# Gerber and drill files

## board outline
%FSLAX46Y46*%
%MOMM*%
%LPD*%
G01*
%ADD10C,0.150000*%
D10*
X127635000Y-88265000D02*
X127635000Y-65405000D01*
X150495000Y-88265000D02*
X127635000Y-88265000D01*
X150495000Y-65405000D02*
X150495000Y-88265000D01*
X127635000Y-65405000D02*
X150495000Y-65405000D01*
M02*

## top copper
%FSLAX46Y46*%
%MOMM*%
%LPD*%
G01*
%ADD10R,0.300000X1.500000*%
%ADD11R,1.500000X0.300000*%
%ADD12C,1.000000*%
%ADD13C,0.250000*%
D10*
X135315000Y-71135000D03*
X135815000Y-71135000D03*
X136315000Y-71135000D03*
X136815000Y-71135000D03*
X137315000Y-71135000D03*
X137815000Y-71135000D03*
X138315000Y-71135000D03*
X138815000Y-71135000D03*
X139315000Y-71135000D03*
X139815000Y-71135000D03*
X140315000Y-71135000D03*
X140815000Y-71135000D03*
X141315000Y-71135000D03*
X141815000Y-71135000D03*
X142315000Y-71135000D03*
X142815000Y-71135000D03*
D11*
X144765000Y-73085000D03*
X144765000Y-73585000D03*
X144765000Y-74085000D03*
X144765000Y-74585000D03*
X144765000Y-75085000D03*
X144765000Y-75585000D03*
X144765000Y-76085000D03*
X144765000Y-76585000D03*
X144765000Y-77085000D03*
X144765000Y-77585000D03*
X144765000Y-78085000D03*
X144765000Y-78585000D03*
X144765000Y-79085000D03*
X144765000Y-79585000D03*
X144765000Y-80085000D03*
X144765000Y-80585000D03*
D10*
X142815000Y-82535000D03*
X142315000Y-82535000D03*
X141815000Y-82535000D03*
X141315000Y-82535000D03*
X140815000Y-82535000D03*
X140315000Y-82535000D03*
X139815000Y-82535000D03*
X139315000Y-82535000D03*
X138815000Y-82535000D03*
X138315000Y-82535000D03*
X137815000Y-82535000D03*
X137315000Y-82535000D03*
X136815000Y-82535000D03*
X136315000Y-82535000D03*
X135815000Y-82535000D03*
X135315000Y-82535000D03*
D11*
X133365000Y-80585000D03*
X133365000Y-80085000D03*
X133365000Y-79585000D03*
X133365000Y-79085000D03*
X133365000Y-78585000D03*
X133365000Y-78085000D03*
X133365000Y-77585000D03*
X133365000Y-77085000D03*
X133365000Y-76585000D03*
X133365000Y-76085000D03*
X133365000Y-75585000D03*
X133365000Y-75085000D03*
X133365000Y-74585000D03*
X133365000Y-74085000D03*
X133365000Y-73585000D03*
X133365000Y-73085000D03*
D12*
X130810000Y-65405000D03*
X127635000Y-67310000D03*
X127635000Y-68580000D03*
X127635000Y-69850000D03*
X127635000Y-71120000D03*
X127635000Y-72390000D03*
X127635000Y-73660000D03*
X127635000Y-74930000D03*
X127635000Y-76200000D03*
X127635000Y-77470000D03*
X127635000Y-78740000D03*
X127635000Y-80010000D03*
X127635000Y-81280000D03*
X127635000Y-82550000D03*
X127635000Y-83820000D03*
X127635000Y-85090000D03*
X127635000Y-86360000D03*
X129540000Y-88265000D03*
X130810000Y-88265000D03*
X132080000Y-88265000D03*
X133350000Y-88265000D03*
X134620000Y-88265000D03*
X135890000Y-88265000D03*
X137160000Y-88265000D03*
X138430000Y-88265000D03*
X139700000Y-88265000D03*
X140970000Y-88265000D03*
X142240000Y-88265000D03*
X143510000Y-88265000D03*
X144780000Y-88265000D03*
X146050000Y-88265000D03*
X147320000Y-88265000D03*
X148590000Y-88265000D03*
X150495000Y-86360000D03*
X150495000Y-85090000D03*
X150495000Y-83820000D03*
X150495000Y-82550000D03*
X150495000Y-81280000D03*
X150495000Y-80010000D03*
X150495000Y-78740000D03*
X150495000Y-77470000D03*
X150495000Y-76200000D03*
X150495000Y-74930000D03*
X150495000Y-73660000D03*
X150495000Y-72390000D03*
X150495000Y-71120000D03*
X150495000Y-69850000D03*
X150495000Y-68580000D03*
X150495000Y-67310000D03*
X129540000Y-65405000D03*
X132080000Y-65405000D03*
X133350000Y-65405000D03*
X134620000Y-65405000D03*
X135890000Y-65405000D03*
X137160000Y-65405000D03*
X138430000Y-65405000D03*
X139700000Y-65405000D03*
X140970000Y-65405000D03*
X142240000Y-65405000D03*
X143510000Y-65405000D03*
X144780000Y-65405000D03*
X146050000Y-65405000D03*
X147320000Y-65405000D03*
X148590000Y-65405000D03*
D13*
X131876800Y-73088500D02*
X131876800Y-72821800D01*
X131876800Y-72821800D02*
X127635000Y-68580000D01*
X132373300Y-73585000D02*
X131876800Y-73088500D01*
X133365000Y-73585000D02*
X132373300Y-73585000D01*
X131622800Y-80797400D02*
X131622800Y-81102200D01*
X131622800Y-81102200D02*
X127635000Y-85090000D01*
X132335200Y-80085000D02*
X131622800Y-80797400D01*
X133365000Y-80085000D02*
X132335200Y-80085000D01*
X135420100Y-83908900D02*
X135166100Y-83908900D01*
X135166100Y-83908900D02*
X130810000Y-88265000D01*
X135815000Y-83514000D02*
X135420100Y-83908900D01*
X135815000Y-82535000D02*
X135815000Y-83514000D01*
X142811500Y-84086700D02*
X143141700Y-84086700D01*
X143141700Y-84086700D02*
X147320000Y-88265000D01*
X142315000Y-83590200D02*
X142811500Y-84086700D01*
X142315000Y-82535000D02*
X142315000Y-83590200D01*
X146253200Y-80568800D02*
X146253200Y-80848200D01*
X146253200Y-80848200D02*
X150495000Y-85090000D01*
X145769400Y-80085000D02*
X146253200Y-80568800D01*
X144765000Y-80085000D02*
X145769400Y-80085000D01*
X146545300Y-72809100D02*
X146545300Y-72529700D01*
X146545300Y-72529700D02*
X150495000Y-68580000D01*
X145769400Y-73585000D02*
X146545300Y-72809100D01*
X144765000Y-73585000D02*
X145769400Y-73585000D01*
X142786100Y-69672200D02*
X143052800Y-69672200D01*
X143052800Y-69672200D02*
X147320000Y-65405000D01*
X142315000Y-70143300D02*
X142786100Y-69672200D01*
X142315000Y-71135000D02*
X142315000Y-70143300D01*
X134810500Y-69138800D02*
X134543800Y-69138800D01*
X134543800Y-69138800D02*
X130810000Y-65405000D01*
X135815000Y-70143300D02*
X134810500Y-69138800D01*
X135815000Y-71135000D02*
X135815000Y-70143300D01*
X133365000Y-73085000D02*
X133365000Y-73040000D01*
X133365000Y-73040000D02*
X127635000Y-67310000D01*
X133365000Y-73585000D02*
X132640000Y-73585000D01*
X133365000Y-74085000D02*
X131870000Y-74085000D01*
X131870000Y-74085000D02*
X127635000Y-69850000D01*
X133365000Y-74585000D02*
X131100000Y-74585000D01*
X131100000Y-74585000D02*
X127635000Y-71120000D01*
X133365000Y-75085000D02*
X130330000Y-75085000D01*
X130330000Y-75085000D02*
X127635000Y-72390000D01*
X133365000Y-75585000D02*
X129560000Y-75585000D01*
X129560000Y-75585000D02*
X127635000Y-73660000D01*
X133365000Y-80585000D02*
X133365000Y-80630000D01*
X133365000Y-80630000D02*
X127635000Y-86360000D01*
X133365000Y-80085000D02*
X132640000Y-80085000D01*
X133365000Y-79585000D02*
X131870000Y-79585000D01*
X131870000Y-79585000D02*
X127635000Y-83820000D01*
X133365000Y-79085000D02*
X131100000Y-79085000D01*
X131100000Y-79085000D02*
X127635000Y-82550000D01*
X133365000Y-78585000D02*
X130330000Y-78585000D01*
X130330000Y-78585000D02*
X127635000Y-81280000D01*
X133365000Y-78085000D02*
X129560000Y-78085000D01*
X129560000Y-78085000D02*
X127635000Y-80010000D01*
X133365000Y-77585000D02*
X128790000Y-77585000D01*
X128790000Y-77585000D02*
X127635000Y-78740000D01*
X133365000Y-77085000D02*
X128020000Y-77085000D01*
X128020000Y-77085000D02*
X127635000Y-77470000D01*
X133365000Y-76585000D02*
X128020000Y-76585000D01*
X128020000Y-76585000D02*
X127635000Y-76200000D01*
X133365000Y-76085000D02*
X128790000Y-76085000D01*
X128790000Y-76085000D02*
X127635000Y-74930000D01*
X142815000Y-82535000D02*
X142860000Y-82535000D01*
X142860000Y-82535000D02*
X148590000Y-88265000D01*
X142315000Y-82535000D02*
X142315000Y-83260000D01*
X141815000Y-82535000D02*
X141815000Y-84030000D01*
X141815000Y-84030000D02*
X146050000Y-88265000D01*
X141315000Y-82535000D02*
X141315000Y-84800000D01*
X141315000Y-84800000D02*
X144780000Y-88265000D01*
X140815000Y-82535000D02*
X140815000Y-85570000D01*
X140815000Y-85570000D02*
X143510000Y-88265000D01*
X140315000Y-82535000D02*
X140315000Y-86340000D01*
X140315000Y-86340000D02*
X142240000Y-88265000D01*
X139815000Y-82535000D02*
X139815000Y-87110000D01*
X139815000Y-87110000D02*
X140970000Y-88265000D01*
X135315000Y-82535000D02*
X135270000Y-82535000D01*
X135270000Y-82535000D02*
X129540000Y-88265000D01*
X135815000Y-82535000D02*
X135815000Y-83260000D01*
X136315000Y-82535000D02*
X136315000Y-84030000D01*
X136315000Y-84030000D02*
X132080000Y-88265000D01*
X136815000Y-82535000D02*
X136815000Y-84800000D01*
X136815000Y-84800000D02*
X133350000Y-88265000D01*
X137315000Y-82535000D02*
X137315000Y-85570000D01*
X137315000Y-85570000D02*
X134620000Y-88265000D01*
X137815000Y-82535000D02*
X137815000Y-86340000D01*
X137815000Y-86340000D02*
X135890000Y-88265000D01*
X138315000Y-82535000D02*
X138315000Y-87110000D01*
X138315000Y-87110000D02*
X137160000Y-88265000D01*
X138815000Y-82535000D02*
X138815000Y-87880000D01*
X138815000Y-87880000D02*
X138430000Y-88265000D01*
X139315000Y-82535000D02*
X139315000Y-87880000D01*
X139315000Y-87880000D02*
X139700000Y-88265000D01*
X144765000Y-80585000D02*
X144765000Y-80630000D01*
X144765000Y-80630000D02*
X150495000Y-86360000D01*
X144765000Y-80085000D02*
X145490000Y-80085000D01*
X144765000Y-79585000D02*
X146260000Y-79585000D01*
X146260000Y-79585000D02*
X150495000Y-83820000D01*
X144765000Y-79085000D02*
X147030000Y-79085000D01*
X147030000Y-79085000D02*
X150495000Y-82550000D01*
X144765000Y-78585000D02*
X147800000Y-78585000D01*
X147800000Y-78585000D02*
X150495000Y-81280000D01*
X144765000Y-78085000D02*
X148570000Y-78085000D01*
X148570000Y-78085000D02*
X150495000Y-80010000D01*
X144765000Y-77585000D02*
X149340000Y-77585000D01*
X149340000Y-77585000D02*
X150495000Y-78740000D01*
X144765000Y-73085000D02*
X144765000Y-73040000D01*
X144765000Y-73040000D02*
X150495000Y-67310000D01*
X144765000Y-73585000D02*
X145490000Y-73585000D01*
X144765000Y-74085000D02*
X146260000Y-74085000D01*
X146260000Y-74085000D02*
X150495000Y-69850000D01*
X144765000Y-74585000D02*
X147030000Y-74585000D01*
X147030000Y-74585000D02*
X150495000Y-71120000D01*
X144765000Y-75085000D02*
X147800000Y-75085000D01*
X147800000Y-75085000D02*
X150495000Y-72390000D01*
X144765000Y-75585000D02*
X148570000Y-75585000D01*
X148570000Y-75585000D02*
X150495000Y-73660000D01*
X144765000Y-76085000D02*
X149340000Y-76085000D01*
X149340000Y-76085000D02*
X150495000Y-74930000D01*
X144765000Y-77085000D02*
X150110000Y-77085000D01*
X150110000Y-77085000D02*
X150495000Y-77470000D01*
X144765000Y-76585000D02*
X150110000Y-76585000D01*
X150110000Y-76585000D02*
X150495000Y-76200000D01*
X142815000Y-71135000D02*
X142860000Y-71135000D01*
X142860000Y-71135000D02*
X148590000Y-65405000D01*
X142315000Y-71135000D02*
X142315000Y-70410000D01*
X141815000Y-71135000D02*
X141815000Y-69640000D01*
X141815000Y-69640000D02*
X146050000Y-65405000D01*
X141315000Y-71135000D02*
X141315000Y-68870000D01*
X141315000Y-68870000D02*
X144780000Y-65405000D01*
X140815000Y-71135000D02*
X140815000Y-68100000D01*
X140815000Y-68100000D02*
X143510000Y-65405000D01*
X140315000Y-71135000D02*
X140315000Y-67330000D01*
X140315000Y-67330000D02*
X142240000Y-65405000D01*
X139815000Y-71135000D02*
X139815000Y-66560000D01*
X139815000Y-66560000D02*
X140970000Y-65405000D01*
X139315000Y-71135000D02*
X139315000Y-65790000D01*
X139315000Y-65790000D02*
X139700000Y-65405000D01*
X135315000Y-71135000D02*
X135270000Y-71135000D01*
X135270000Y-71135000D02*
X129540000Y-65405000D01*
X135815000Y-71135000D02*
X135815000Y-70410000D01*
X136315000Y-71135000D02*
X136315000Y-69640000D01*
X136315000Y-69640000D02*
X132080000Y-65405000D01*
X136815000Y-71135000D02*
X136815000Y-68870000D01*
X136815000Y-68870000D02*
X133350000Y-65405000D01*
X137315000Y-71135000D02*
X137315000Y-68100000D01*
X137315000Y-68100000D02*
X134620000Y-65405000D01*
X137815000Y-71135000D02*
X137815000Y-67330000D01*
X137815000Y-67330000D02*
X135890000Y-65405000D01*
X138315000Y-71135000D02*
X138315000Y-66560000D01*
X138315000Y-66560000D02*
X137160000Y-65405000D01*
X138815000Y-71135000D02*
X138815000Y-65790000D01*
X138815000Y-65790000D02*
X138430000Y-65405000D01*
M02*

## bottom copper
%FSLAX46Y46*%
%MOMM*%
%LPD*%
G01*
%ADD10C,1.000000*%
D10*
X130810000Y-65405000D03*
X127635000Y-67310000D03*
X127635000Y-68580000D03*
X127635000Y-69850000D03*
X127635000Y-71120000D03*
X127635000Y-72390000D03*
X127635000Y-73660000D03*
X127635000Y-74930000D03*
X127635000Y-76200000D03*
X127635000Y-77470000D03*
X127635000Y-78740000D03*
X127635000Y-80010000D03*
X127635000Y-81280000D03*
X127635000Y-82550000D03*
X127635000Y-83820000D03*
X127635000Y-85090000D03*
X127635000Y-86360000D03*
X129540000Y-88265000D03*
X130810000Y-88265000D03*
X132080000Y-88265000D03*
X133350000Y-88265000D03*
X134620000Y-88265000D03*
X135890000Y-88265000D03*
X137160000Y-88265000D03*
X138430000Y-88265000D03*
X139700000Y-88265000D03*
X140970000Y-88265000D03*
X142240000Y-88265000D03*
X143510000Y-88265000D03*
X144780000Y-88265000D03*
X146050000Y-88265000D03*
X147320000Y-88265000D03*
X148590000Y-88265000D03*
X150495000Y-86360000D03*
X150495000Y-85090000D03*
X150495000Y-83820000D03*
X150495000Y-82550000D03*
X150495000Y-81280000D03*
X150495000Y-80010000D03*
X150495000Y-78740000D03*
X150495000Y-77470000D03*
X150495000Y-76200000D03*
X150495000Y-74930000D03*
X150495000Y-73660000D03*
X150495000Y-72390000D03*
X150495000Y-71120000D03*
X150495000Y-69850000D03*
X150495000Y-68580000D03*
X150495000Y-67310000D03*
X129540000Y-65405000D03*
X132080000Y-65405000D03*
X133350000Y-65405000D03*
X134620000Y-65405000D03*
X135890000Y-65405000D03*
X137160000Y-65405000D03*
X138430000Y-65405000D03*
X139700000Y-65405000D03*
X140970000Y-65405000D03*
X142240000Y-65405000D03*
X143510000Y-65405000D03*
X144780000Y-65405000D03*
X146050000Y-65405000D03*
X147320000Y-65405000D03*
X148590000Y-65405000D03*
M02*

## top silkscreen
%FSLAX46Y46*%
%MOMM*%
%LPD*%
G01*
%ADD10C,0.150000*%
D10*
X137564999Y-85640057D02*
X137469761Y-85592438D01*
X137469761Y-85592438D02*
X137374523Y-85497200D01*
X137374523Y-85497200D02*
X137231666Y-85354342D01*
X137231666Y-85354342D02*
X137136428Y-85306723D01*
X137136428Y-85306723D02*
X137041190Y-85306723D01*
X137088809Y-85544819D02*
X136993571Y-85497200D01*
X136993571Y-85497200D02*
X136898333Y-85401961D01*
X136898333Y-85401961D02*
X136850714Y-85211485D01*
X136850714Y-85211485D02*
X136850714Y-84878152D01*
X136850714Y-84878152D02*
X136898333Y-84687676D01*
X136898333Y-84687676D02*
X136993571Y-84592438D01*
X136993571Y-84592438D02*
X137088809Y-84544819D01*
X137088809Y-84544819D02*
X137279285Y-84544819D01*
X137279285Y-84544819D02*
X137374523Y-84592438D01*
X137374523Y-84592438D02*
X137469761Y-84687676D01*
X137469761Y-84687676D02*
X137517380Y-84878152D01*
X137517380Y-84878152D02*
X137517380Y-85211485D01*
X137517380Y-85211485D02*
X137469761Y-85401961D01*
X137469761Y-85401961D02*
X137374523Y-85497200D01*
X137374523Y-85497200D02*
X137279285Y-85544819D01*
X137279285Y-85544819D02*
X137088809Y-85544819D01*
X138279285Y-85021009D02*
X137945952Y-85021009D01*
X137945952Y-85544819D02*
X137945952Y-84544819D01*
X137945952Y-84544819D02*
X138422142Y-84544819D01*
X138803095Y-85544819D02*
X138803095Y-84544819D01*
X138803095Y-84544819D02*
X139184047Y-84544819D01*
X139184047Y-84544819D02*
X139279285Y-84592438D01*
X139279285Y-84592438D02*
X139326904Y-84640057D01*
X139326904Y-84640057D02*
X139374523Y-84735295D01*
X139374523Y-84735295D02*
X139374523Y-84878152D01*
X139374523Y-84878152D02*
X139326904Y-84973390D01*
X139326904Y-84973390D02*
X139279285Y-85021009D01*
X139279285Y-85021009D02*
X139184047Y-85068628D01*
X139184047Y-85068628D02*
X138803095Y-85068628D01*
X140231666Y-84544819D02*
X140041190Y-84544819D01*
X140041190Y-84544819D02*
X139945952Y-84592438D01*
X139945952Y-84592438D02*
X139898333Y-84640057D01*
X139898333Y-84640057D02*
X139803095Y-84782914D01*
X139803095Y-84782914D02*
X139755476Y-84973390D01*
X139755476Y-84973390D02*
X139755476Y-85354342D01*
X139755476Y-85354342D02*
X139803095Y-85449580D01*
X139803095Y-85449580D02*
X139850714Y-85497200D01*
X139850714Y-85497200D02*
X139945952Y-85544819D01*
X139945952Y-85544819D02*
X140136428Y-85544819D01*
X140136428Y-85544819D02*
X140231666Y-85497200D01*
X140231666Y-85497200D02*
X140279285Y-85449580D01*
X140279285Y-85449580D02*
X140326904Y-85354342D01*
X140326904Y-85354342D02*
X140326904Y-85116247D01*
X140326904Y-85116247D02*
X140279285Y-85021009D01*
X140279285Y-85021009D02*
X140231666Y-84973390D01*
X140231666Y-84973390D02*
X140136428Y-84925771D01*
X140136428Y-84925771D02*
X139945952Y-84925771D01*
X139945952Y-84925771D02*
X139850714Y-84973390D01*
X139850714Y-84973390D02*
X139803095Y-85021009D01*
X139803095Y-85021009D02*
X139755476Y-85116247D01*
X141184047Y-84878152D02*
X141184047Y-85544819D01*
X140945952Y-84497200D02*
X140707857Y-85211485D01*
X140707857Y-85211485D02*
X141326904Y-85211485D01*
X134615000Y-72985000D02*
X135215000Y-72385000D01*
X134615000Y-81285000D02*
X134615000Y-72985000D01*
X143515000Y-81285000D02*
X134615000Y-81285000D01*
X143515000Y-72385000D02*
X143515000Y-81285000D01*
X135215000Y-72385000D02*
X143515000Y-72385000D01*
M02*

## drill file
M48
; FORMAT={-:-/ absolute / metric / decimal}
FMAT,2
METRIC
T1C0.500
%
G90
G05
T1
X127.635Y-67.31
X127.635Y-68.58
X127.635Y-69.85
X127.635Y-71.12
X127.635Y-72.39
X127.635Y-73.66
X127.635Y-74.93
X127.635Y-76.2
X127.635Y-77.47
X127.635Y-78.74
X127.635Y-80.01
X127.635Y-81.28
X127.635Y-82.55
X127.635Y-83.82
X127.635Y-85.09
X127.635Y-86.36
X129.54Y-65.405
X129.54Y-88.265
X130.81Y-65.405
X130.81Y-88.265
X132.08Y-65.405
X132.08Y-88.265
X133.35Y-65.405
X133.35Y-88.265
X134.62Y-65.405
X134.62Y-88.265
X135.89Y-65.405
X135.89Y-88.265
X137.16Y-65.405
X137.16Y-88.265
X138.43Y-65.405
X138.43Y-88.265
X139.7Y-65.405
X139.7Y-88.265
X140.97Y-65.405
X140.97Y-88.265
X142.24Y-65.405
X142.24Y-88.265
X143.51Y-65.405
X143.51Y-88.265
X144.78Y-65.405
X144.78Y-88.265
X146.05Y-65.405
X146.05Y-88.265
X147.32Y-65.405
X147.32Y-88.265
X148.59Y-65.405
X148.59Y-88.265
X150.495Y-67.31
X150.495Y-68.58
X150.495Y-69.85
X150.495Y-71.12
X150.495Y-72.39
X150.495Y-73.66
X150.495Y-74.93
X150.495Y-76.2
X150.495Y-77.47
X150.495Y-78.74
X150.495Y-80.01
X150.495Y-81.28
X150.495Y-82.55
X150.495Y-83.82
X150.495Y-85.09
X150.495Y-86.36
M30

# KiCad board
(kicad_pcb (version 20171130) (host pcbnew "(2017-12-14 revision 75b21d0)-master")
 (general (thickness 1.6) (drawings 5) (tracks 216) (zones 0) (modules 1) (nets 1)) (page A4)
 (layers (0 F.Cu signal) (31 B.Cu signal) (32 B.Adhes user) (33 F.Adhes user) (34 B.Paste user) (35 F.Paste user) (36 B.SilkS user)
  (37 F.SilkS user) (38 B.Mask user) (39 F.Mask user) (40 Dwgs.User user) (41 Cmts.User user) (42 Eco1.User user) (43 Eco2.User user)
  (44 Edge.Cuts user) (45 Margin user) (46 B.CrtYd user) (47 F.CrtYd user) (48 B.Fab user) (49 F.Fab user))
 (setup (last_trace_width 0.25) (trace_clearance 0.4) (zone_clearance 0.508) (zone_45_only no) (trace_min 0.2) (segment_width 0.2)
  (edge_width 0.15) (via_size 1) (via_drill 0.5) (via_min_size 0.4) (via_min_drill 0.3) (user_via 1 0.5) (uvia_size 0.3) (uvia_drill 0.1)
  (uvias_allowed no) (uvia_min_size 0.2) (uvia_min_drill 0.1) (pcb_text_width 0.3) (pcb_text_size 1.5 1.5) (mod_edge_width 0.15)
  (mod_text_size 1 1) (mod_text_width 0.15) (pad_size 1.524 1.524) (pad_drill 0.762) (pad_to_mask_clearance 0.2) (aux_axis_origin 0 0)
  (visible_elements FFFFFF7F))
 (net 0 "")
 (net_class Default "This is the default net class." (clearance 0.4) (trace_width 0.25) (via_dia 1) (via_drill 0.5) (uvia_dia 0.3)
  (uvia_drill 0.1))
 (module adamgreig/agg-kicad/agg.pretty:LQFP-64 (layer F.Cu) (at 139.065 76.835)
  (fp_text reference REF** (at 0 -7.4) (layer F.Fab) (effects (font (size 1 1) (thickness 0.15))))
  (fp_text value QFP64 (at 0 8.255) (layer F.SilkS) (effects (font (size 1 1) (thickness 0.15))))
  (fp_line (start -4.45 -3.85) (end -3.85 -4.45) (layer F.SilkS) (width 0.15))
  (fp_line (start -4.45 4.45) (end -4.45 -3.85) (layer F.SilkS) (width 0.15))
  (fp_line (start 4.45 4.45) (end -4.45 4.45) (layer F.SilkS) (width 0.15))
  (fp_line (start 4.45 -4.45) (end 4.45 4.45) (layer F.SilkS) (width 0.15))
  (fp_line (start -3.85 -4.45) (end 4.45 -4.45) (layer F.SilkS) (width 0.15))
  (pad 64 smd rect (at -3.75 -5.7) (size 0.3 1.5) (layers F.Cu F.Paste F.Mask))
  (pad 63 smd rect (at -3.25 -5.7) (size 0.3 1.5) (layers F.Cu F.Paste F.Mask))
  (pad 62 smd rect (at -2.75 -5.7) (size 0.3 1.5) (layers F.Cu F.Paste F.Mask))
  (pad 61 smd rect (at -2.25 -5.7) (size 0.3 1.5) (layers F.Cu F.Paste F.Mask))
  (pad 60 smd rect (at -1.75 -5.7) (size 0.3 1.5) (layers F.Cu F.Paste F.Mask))
  (pad 59 smd rect (at -1.25 -5.7) (size 0.3 1.5) (layers F.Cu F.Paste F.Mask))
  (pad 58 smd rect (at -0.75 -5.7) (size 0.3 1.5) (layers F.Cu F.Paste F.Mask))
  (pad 57 smd rect (at -0.25 -5.7) (size 0.3 1.5) (layers F.Cu F.Paste F.Mask))
  (pad 56 smd rect (at 0.25 -5.7) (size 0.3 1.5) (layers F.Cu F.Paste F.Mask))
  (pad 55 smd rect (at 0.75 -5.7) (size 0.3 1.5) (layers F.Cu F.Paste F.Mask))
  (pad 54 smd rect (at 1.25 -5.7) (size 0.3 1.5) (layers F.Cu F.Paste F.Mask))
  (pad 53 smd rect (at 1.75 -5.7) (size 0.3 1.5) (layers F.Cu F.Paste F.Mask))
  (pad 52 smd rect (at 2.25 -5.7) (size 0.3 1.5) (layers F.Cu F.Paste F.Mask))
  (pad 51 smd rect (at 2.75 -5.7) (size 0.3 1.5) (layers F.Cu F.Paste F.Mask))
  (pad 50 smd rect (at 3.25 -5.7) (size 0.3 1.5) (layers F.Cu F.Paste F.Mask))
  (pad 49 smd rect (at 3.75 -5.7) (size 0.3 1.5) (layers F.Cu F.Paste F.Mask))
  (pad 48 smd rect (at 5.7 -3.75) (size 1.5 0.3) (layers F.Cu F.Paste F.Mask))
  (pad 47 smd rect (at 5.7 -3.25) (size 1.5 0.3) (layers F.Cu F.Paste F.Mask))
  (pad 46 smd rect (at 5.7 -2.75) (size 1.5 0.3) (layers F.Cu F.Paste F.Mask))
  (pad 45 smd rect (at 5.7 -2.25) (size 1.5 0.3) (layers F.Cu F.Paste F.Mask))
  (pad 44 smd rect (at 5.7 -1.75) (size 1.5 0.3) (layers F.Cu F.Paste F.Mask))
  (pad 43 smd rect (at 5.7 -1.25) (size 1.5 0.3) (layers F.Cu F.Paste F.Mask))
  (pad 42 smd rect (at 5.7 -0.75) (size 1.5 0.3) (layers F.Cu F.Paste F.Mask))
  (pad 41 smd rect (at 5.7 -0.25) (size 1.5 0.3) (layers F.Cu F.Paste F.Mask))
  (pad 40 smd rect (at 5.7 0.25) (size 1.5 0.3) (layers F.Cu F.Paste F.Mask))
  (pad 39 smd rect (at 5.7 0.75) (size 1.5 0.3) (layers F.Cu F.Paste F.Mask))
  (pad 38 smd rect (at 5.7 1.25) (size 1.5 0.3) (layers F.Cu F.Paste F.Mask))
  (pad 37 smd rect (at 5.7 1.75) (size 1.5 0.3) (layers F.Cu F.Paste F.Mask))
  (pad 36 smd rect (at 5.7 2.25) (size 1.5 0.3) (layers F.Cu F.Paste F.Mask))
  (pad 35 smd rect (at 5.7 2.75) (size 1.5 0.3) (layers F.Cu F.Paste F.Mask))
  (pad 34 smd rect (at 5.7 3.25) (size 1.5 0.3) (layers F.Cu F.Paste F.Mask))
  (pad 33 smd rect (at 5.7 3.75) (size 1.5 0.3) (layers F.Cu F.Paste F.Mask))
  (pad 32 smd rect (at 3.75 5.7) (size 0.3 1.5) (layers F.Cu F.Paste F.Mask))
  (pad 31 smd rect (at 3.25 5.7) (size 0.3 1.5) (layers F.Cu F.Paste F.Mask))
  (pad 30 smd rect (at 2.75 5.7) (size 0.3 1.5) (layers F.Cu F.Paste F.Mask))
  (pad 29 smd rect (at 2.25 5.7) (size 0.3 1.5) (layers F.Cu F.Paste F.Mask))
  (pad 28 smd rect (at 1.75 5.7) (size 0.3 1.5) (layers F.Cu F.Paste F.Mask))
  (pad 27 smd rect (at 1.25 5.7) (size 0.3 1.5) (layers F.Cu F.Paste F.Mask))
  (pad 26 smd rect (at 0.75 5.7) (size 0.3 1.5) (layers F.Cu F.Paste F.Mask))
  (pad 25 smd rect (at 0.25 5.7) (size 0.3 1.5) (layers F.Cu F.Paste F.Mask))
  (pad 24 smd rect (at -0.25 5.7) (size 0.3 1.5) (layers F.Cu F.Paste F.Mask))
  (pad 23 smd rect (at -0.75 5.7) (size 0.3 1.5) (layers F.Cu F.Paste F.Mask))
  (pad 22 smd rect (at -1.25 5.7) (size 0.3 1.5) (layers F.Cu F.Paste F.Mask))
  (pad 21 smd rect (at -1.75 5.7) (size 0.3 1.5) (layers F.Cu F.Paste F.Mask))
  (pad 20 smd rect (at -2.25 5.7) (size 0.3 1.5) (layers F.Cu F.Paste F.Mask))
  (pad 19 smd rect (at -2.75 5.7) (size 0.3 1.5) (layers F.Cu F.Paste F.Mask))
  (pad 18 smd rect (at -3.25 5.7) (size 0.3 1.5) (layers F.Cu F.Paste F.Mask))
  (pad 17 smd rect (at -3.75 5.7) (size 0.3 1.5) (layers F.Cu F.Paste F.Mask))
  (pad 16 smd rect (at -5.7 3.75) (size 1.5 0.3) (layers F.Cu F.Paste F.Mask))
  (pad 15 smd rect (at -5.7 3.25) (size 1.5 0.3) (layers F.Cu F.Paste F.Mask))
  (pad 14 smd rect (at -5.7 2.75) (size 1.5 0.3) (layers F.Cu F.Paste F.Mask))
  (pad 13 smd rect (at -5.7 2.25) (size 1.5 0.3) (layers F.Cu F.Paste F.Mask))
  (pad 12 smd rect (at -5.7 1.75) (size 1.5 0.3) (layers F.Cu F.Paste F.Mask))
  (pad 11 smd rect (at -5.7 1.25) (size 1.5 0.3) (layers F.Cu F.Paste F.Mask))
  (pad 10 smd rect (at -5.7 0.75) (size 1.5 0.3) (layers F.Cu F.Paste F.Mask))
  (pad 9 smd rect (at -5.7 0.25) (size 1.5 0.3) (layers F.Cu F.Paste F.Mask))
  (pad 8 smd rect (at -5.7 -0.25) (size 1.5 0.3) (layers F.Cu F.Paste F.Mask))
  (pad 7 smd rect (at -5.7 -0.75) (size 1.5 0.3) (layers F.Cu F.Paste F.Mask))
  (pad 6 smd rect (at -5.7 -1.25) (size 1.5 0.3) (layers F.Cu F.Paste F.Mask))
  (pad 5 smd rect (at -5.7 -1.75) (size 1.5 0.3) (layers F.Cu F.Paste F.Mask))
  (pad 4 smd rect (at -5.7 -2.25) (size 1.5 0.3) (layers F.Cu F.Paste F.Mask))
  (pad 3 smd rect (at -5.7 -2.75) (size 1.5 0.3) (layers F.Cu F.Paste F.Mask))
  (pad 2 smd rect (at -5.7 -3.25) (size 1.5 0.3) (layers F.Cu F.Paste F.Mask))
  (pad 1 smd rect (at -5.7 -3.75) (size 1.5 0.3) (layers F.Cu F.Paste F.Mask)))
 (gr_line (start 127.635 88.265) (end 127.635 65.405) (layer Edge.Cuts) (width 0.15))
 (gr_line (start 150.495 88.265) (end 127.635 88.265) (layer Edge.Cuts) (width 0.15))
 (gr_line (start 150.495 65.405) (end 150.495 88.265) (layer Edge.Cuts) (width 0.15))
 (gr_line (start 127.635 65.405) (end 150.495 65.405) (layer Edge.Cuts) (width 0.15))
 (segment (start 131.8768 73.0885) (end 131.8768 72.8218) (width 0.25) (layer F.Cu) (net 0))
 (segment (start 131.8768 72.8218) (end 127.635 68.58) (width 0.25) (layer F.Cu) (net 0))
 (segment (start 132.3733 73.585) (end 131.8768 73.0885) (width 0.25) (layer F.Cu) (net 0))
 (segment (start 133.365 73.585) (end 132.3733 73.585) (width 0.25) (layer F.Cu) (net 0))
 (segment (start 131.6228 80.7974) (end 131.6228 81.1022) (width 0.25) (layer F.Cu) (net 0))
 (segment (start 131.6228 81.1022) (end 127.635 85.09) (width 0.25) (layer F.Cu) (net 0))
 (segment (start 132.3352 80.085) (end 131.6228 80.7974) (width 0.25) (layer F.Cu) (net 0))
 (segment (start 133.365 80.085) (end 132.3352 80.085) (width 0.25) (layer F.Cu) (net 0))
 (segment (start 135.4201 83.9089) (end 135.1661 83.9089) (width 0.25) (layer F.Cu) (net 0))
 (segment (start 135.1661 83.9089) (end 130.81 88.265) (width 0.25) (layer F.Cu) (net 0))
 (segment (start 135.815 83.514) (end 135.4201 83.9089) (width 0.25) (layer F.Cu) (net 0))
 (segment (start 135.815 82.535) (end 135.815 83.514) (width 0.25) (layer F.Cu) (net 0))
 (segment (start 142.8115 84.0867) (end 143.1417 84.0867) (width 0.25) (layer F.Cu) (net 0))
 (segment (start 143.1417 84.0867) (end 147.32 88.265) (width 0.25) (layer F.Cu) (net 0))
 (segment (start 142.315 83.5902) (end 142.8115 84.0867) (width 0.25) (layer F.Cu) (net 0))
 (segment (start 142.315 82.535) (end 142.315 83.5902) (width 0.25) (layer F.Cu) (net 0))
 (segment (start 146.2532 80.5688) (end 146.2532 80.8482) (width 0.25) (layer F.Cu) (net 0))
 (segment (start 146.2532 80.8482) (end 150.495 85.09) (width 0.25) (layer F.Cu) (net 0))
 (segment (start 145.7694 80.085) (end 146.2532 80.5688) (width 0.25) (layer F.Cu) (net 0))
 (segment (start 144.765 80.085) (end 145.7694 80.085) (width 0.25) (layer F.Cu) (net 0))
 (segment (start 146.5453 72.8091) (end 146.5453 72.5297) (width 0.25) (layer F.Cu) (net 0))
 (segment (start 146.5453 72.5297) (end 150.495 68.58) (width 0.25) (layer F.Cu) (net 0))
 (segment (start 145.7694 73.585) (end 146.5453 72.8091) (width 0.25) (layer F.Cu) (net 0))
 (segment (start 144.765 73.585) (end 145.7694 73.585) (width 0.25) (layer F.Cu) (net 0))
 (segment (start 142.7861 69.6722) (end 143.0528 69.6722) (width 0.25) (layer F.Cu) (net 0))
 (segment (start 143.0528 69.6722) (end 147.32 65.405) (width 0.25) (layer F.Cu) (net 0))
 (segment (start 142.315 70.1433) (end 142.7861 69.6722) (width 0.25) (layer F.Cu) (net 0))
 (segment (start 142.315 71.135) (end 142.315 70.1433) (width 0.25) (layer F.Cu) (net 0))
 (segment (start 134.8105 69.1388) (end 134.5438 69.1388) (width 0.25) (layer F.Cu) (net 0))
 (segment (start 134.5438 69.1388) (end 130.81 65.405) (width 0.25) (layer F.Cu) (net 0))
 (segment (start 135.815 70.1433) (end 134.8105 69.1388) (width 0.25) (layer F.Cu) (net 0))
 (segment (start 135.815 71.135) (end 135.815 70.1433) (width 0.25) (layer F.Cu) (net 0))
 (segment (start 133.365 73.085) (end 133.365 73.04) (width 0.25) (layer F.Cu) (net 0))
 (segment (start 133.365 73.04) (end 127.635 67.31) (width 0.25) (layer F.Cu) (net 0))
 (segment (start 133.365 73.585) (end 132.64 73.585) (width 0.25) (layer F.Cu) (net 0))
 (segment (start 133.365 74.085) (end 131.87 74.085) (width 0.25) (layer F.Cu) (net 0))
 (segment (start 131.87 74.085) (end 127.635 69.85) (width 0.25) (layer F.Cu) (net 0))
 (segment (start 133.365 74.585) (end 131.1 74.585) (width 0.25) (layer F.Cu) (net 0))
 (segment (start 131.1 74.585) (end 127.635 71.12) (width 0.25) (layer F.Cu) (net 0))
 (segment (start 133.365 75.085) (end 130.33 75.085) (width 0.25) (layer F.Cu) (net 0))
 (segment (start 130.33 75.085) (end 127.635 72.39) (width 0.25) (layer F.Cu) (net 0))
 (segment (start 133.365 75.585) (end 129.56 75.585) (width 0.25) (layer F.Cu) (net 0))
 (segment (start 129.56 75.585) (end 127.635 73.66) (width 0.25) (layer F.Cu) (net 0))
 (segment (start 133.365 80.585) (end 133.365 80.63) (width 0.25) (layer F.Cu) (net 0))
 (segment (start 133.365 80.63) (end 127.635 86.36) (width 0.25) (layer F.Cu) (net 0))
 (segment (start 133.365 80.085) (end 132.64 80.085) (width 0.25) (layer F.Cu) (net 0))
 (segment (start 133.365 79.585) (end 131.87 79.585) (width 0.25) (layer F.Cu) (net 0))
 (segment (start 131.87 79.585) (end 127.635 83.82) (width 0.25) (layer F.Cu) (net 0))
 (segment (start 133.365 79.085) (end 131.1 79.085) (width 0.25) (layer F.Cu) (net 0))
 (segment (start 131.1 79.085) (end 127.635 82.55) (width 0.25) (layer F.Cu) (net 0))
 (segment (start 133.365 78.585) (end 130.33 78.585) (width 0.25) (layer F.Cu) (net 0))
 (segment (start 130.33 78.585) (end 127.635 81.28) (width 0.25) (layer F.Cu) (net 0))
 (segment (start 133.365 78.085) (end 129.56 78.085) (width 0.25) (layer F.Cu) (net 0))
 (segment (start 129.56 78.085) (end 127.635 80.01) (width 0.25) (layer F.Cu) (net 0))
 (segment (start 133.365 77.585) (end 128.79 77.585) (width 0.25) (layer F.Cu) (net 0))
 (segment (start 128.79 77.585) (end 127.635 78.74) (width 0.25) (layer F.Cu) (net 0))
 (segment (start 133.365 77.085) (end 128.02 77.085) (width 0.25) (layer F.Cu) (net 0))
 (segment (start 128.02 77.085) (end 127.635 77.47) (width 0.25) (layer F.Cu) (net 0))
 (segment (start 133.365 76.585) (end 128.02 76.585) (width 0.25) (layer F.Cu) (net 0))
 (segment (start 128.02 76.585) (end 127.635 76.2) (width 0.25) (layer F.Cu) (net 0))
 (segment (start 133.365 76.085) (end 128.79 76.085) (width 0.25) (layer F.Cu) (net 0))
 (segment (start 128.79 76.085) (end 127.635 74.93) (width 0.25) (layer F.Cu) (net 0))
 (segment (start 142.815 82.535) (end 142.86 82.535) (width 0.25) (layer F.Cu) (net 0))
 (segment (start 142.86 82.535) (end 148.59 88.265) (width 0.25) (layer F.Cu) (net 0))
 (segment (start 142.315 82.535) (end 142.315 83.26) (width 0.25) (layer F.Cu) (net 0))
 (segment (start 141.815 82.535) (end 141.815 84.03) (width 0.25) (layer F.Cu) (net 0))
 (segment (start 141.815 84.03) (end 146.05 88.265) (width 0.25) (layer F.Cu) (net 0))
 (segment (start 141.315 82.535) (end 141.315 84.8) (width 0.25) (layer F.Cu) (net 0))
 (segment (start 141.315 84.8) (end 144.78 88.265) (width 0.25) (layer F.Cu) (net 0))
 (segment (start 140.815 82.535) (end 140.815 85.57) (width 0.25) (layer F.Cu) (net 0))
 (segment (start 140.815 85.57) (end 143.51 88.265) (width 0.25) (layer F.Cu) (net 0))
 (segment (start 140.315 82.535) (end 140.315 86.34) (width 0.25) (layer F.Cu) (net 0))
 (segment (start 140.315 86.34) (end 142.24 88.265) (width 0.25) (layer F.Cu) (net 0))
 (segment (start 139.815 82.535) (end 139.815 87.11) (width 0.25) (layer F.Cu) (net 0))
 (segment (start 139.815 87.11) (end 140.97 88.265) (width 0.25) (layer F.Cu) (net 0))
 (segment (start 135.315 82.535) (end 135.27 82.535) (width 0.25) (layer F.Cu) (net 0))
 (segment (start 135.27 82.535) (end 129.54 88.265) (width 0.25) (layer F.Cu) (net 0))
 (segment (start 135.815 82.535) (end 135.815 83.26) (width 0.25) (layer F.Cu) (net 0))
 (segment (start 136.315 82.535) (end 136.315 84.03) (width 0.25) (layer F.Cu) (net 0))
 (segment (start 136.315 84.03) (end 132.08 88.265) (width 0.25) (layer F.Cu) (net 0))
 (segment (start 136.815 82.535) (end 136.815 84.8) (width 0.25) (layer F.Cu) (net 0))
 (segment (start 136.815 84.8) (end 133.35 88.265) (width 0.25) (layer F.Cu) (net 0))
 (segment (start 137.315 82.535) (end 137.315 85.57) (width 0.25) (layer F.Cu) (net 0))
 (segment (start 137.315 85.57) (end 134.62 88.265) (width 0.25) (layer F.Cu) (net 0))
 (segment (start 137.815 82.535) (end 137.815 86.34) (width 0.25) (layer F.Cu) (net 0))
 (segment (start 137.815 86.34) (end 135.89 88.265) (width 0.25) (layer F.Cu) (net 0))
 (segment (start 138.315 82.535) (end 138.315 87.11) (width 0.25) (layer F.Cu) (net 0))
 (segment (start 138.315 87.11) (end 137.16 88.265) (width 0.25) (layer F.Cu) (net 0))
 (segment (start 138.815 82.535) (end 138.815 87.88) (width 0.25) (layer F.Cu) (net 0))
 (segment (start 138.815 87.88) (end 138.43 88.265) (width 0.25) (layer F.Cu) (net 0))
 (segment (start 139.315 82.535) (end 139.315 87.88) (width 0.25) (layer F.Cu) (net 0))
 (segment (start 139.315 87.88) (end 139.7 88.265) (width 0.25) (layer F.Cu) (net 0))
 (segment (start 144.765 80.585) (end 144.765 80.63) (width 0.25) (layer F.Cu) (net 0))
 (segment (start 144.765 80.63) (end 150.495 86.36) (width 0.25) (layer F.Cu) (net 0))
 (segment (start 144.765 80.085) (end 145.49 80.085) (width 0.25) (layer F.Cu) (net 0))
 (segment (start 144.765 79.585) (end 146.26 79.585) (width 0.25) (layer F.Cu) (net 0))
 (segment (start 146.26 79.585) (end 150.495 83.82) (width 0.25) (layer F.Cu) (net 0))
 (segment (start 144.765 79.085) (end 147.03 79.085) (width 0.25) (layer F.Cu) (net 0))
 (segment (start 147.03 79.085) (end 150.495 82.55) (width 0.25) (layer F.Cu) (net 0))
 (segment (start 144.765 78.585) (end 147.8 78.585) (width 0.25) (layer F.Cu) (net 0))
 (segment (start 147.8 78.585) (end 150.495 81.28) (width 0.25) (layer F.Cu) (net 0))
 (segment (start 144.765 78.085) (end 148.57 78.085) (width 0.25) (layer F.Cu) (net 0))
 (segment (start 148.57 78.085) (end 150.495 80.01) (width 0.25) (layer F.Cu) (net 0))
 (segment (start 144.765 77.585) (end 149.34 77.585) (width 0.25) (layer F.Cu) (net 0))
 (segment (start 149.34 77.585) (end 150.495 78.74) (width 0.25) (layer F.Cu) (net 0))
 (segment (start 144.765 73.085) (end 144.765 73.04) (width 0.25) (layer F.Cu) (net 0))
 (segment (start 144.765 73.04) (end 150.495 67.31) (width 0.25) (layer F.Cu) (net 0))
 (segment (start 144.765 73.585) (end 145.49 73.585) (width 0.25) (layer F.Cu) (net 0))
 (segment (start 144.765 74.085) (end 146.26 74.085) (width 0.25) (layer F.Cu) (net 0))
 (segment (start 146.26 74.085) (end 150.495 69.85) (width 0.25) (layer F.Cu) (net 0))
 (segment (start 144.765 74.585) (end 147.03 74.585) (width 0.25) (layer F.Cu) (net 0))
 (segment (start 147.03 74.585) (end 150.495 71.12) (width 0.25) (layer F.Cu) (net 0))
 (segment (start 144.765 75.085) (end 147.8 75.085) (width 0.25) (layer F.Cu) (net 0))
 (segment (start 147.8 75.085) (end 150.495 72.39) (width 0.25) (layer F.Cu) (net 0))
 (segment (start 144.765 75.585) (end 148.57 75.585) (width 0.25) (layer F.Cu) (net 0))
 (segment (start 148.57 75.585) (end 150.495 73.66) (width 0.25) (layer F.Cu) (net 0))
 (segment (start 144.765 76.085) (end 149.34 76.085) (width 0.25) (layer F.Cu) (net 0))
 (segment (start 149.34 76.085) (end 150.495 74.93) (width 0.25) (layer F.Cu) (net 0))
 (segment (start 144.765 77.085) (end 150.11 77.085) (width 0.25) (layer F.Cu) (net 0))
 (segment (start 150.11 77.085) (end 150.495 77.47) (width 0.25) (layer F.Cu) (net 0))
 (segment (start 144.765 76.585) (end 150.11 76.585) (width 0.25) (layer F.Cu) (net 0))
 (segment (start 150.11 76.585) (end 150.495 76.2) (width 0.25) (layer F.Cu) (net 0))
 (segment (start 142.815 71.135) (end 142.86 71.135) (width 0.25) (layer F.Cu) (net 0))
 (segment (start 142.86 71.135) (end 148.59 65.405) (width 0.25) (layer F.Cu) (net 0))
 (segment (start 142.315 71.135) (end 142.315 70.41) (width 0.25) (layer F.Cu) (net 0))
 (segment (start 141.815 71.135) (end 141.815 69.64) (width 0.25) (layer F.Cu) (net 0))
 (segment (start 141.815 69.64) (end 146.05 65.405) (width 0.25) (layer F.Cu) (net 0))
 (segment (start 141.315 71.135) (end 141.315 68.87) (width 0.25) (layer F.Cu) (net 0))
 (segment (start 141.315 68.87) (end 144.78 65.405) (width 0.25) (layer F.Cu) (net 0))
 (segment (start 140.815 71.135) (end 140.815 68.1) (width 0.25) (layer F.Cu) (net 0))
 (segment (start 140.815 68.1) (end 143.51 65.405) (width 0.25) (layer F.Cu) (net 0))
 (segment (start 140.315 71.135) (end 140.315 67.33) (width 0.25) (layer F.Cu) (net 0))
 (segment (start 140.315 67.33) (end 142.24 65.405) (width 0.25) (layer F.Cu) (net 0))
 (segment (start 139.815 71.135) (end 139.815 66.56) (width 0.25) (layer F.Cu) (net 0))
 (segment (start 139.815 66.56) (end 140.97 65.405) (width 0.25) (layer F.Cu) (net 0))
 (segment (start 139.315 71.135) (end 139.315 65.79) (width 0.25) (layer F.Cu) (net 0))
 (segment (start 139.315 65.79) (end 139.7 65.405) (width 0.25) (layer F.Cu) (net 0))
 (segment (start 135.315 71.135) (end 135.27 71.135) (width 0.25) (layer F.Cu) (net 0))
 (segment (start 135.27 71.135) (end 129.54 65.405) (width 0.25) (layer F.Cu) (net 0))
 (segment (start 135.815 71.135) (end 135.815 70.41) (width 0.25) (layer F.Cu) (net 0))
 (via (at 130.81 65.405) (size 1) (drill 0.5) (layers F.Cu B.Cu) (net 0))
 (segment (start 136.315 71.135) (end 136.315 69.64) (width 0.25) (layer F.Cu) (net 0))
 (segment (start 136.315 69.64) (end 132.08 65.405) (width 0.25) (layer F.Cu) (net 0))
 (segment (start 136.815 71.135) (end 136.815 68.87) (width 0.25) (layer F.Cu) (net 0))
 (segment (start 136.815 68.87) (end 133.35 65.405) (width 0.25) (layer F.Cu) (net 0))
 (segment (start 137.315 71.135) (end 137.315 68.1) (width 0.25) (layer F.Cu) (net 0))
 (segment (start 137.315 68.1) (end 134.62 65.405) (width 0.25) (layer F.Cu) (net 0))
 (segment (start 137.815 71.135) (end 137.815 67.33) (width 0.25) (layer F.Cu) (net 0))
 (segment (start 137.815 67.33) (end 135.89 65.405) (width 0.25) (layer F.Cu) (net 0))
 (segment (start 138.315 71.135) (end 138.315 66.56) (width 0.25) (layer F.Cu) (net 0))
 (segment (start 138.315 66.56) (end 137.16 65.405) (width 0.25) (layer F.Cu) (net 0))
 (segment (start 138.815 71.135) (end 138.815 65.79) (width 0.25) (layer F.Cu) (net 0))
 (segment (start 138.815 65.79) (end 138.43 65.405) (width 0.25) (layer F.Cu) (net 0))
 (via (at 127.635 67.31) (size 1) (drill 0.5) (layers F.Cu B.Cu) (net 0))
 (via (at 127.635 68.58) (size 1) (drill 0.5) (layers F.Cu B.Cu) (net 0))
 (via (at 127.635 69.85) (size 1) (drill 0.5) (layers F.Cu B.Cu) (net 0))
 (via (at 127.635 71.12) (size 1) (drill 0.5) (layers F.Cu B.Cu) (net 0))
 (via (at 127.635 72.39) (size 1) (drill 0.5) (layers F.Cu B.Cu) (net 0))
 (via (at 127.635 73.66) (size 1) (drill 0.5) (layers F.Cu B.Cu) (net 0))
 (via (at 127.635 74.93) (size 1) (drill 0.5) (layers F.Cu B.Cu) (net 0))
 (via (at 127.635 76.2) (size 1) (drill 0.5) (layers F.Cu B.Cu) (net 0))
 (via (at 127.635 77.47) (size 1) (drill 0.5) (layers F.Cu B.Cu) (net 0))
 (via (at 127.635 78.74) (size 1) (drill 0.5) (layers F.Cu B.Cu) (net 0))
 (via (at 127.635 80.01) (size 1) (drill 0.5) (layers F.Cu B.Cu) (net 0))
 (via (at 127.635 81.28) (size 1) (drill 0.5) (layers F.Cu B.Cu) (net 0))
 (via (at 127.635 82.55) (size 1) (drill 0.5) (layers F.Cu B.Cu) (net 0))
 (via (at 127.635 83.82) (size 1) (drill 0.5) (layers F.Cu B.Cu) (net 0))
 (via (at 127.635 85.09) (size 1) (drill 0.5) (layers F.Cu B.Cu) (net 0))
 (via (at 127.635 86.36) (size 1) (drill 0.5) (layers F.Cu B.Cu) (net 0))
 (via (at 129.54 88.265) (size 1) (drill 0.5) (layers F.Cu B.Cu) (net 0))
 (via (at 130.81 88.265) (size 1) (drill 0.5) (layers F.Cu B.Cu) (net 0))
 (via (at 132.08 88.265) (size 1) (drill 0.5) (layers F.Cu B.Cu) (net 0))
 (via (at 133.35 88.265) (size 1) (drill 0.5) (layers F.Cu B.Cu) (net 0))
 (via (at 134.62 88.265) (size 1) (drill 0.5) (layers F.Cu B.Cu) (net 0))
 (via (at 135.89 88.265) (size 1) (drill 0.5) (layers F.Cu B.Cu) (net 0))
 (via (at 137.16 88.265) (size 1) (drill 0.5) (layers F.Cu B.Cu) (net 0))
 (via (at 138.43 88.265) (size 1) (drill 0.5) (layers F.Cu B.Cu) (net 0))
 (via (at 139.7 88.265) (size 1) (drill 0.5) (layers F.Cu B.Cu) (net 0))
 (via (at 140.97 88.265) (size 1) (drill 0.5) (layers F.Cu B.Cu) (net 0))
 (via (at 142.24 88.265) (size 1) (drill 0.5) (layers F.Cu B.Cu) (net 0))
 (via (at 143.51 88.265) (size 1) (drill 0.5) (layers F.Cu B.Cu) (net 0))
 (via (at 144.78 88.265) (size 1) (drill 0.5) (layers F.Cu B.Cu) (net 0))
 (via (at 146.05 88.265) (size 1) (drill 0.5) (layers F.Cu B.Cu) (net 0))
 (via (at 147.32 88.265) (size 1) (drill 0.5) (layers F.Cu B.Cu) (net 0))
 (via (at 148.59 88.265) (size 1) (drill 0.5) (layers F.Cu B.Cu) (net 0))
 (via (at 150.495 86.36) (size 1) (drill 0.5) (layers F.Cu B.Cu) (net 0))
 (via (at 150.495 85.09) (size 1) (drill 0.5) (layers F.Cu B.Cu) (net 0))
 (via (at 150.495 83.82) (size 1) (drill 0.5) (layers F.Cu B.Cu) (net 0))
 (via (at 150.495 82.55) (size 1) (drill 0.5) (layers F.Cu B.Cu) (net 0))
 (via (at 150.495 81.28) (size 1) (drill 0.5) (layers F.Cu B.Cu) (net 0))
 (via (at 150.495 80.01) (size 1) (drill 0.5) (layers F.Cu B.Cu) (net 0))
 (via (at 150.495 78.74) (size 1) (drill 0.5) (layers F.Cu B.Cu) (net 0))
 (via (at 150.495 77.47) (size 1) (drill 0.5) (layers F.Cu B.Cu) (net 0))
 (via (at 150.495 76.2) (size 1) (drill 0.5) (layers F.Cu B.Cu) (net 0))
 (via (at 150.495 74.93) (size 1) (drill 0.5) (layers F.Cu B.Cu) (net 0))
 (via (at 150.495 73.66) (size 1) (drill 0.5) (layers F.Cu B.Cu) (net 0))
 (via (at 150.495 72.39) (size 1) (drill 0.5) (layers F.Cu B.Cu) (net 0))
 (via (at 150.495 71.12) (size 1) (drill 0.5) (layers F.Cu B.Cu) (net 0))
 (via (at 150.495 69.85) (size 1) (drill 0.5) (layers F.Cu B.Cu) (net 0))
 (via (at 150.495 68.58) (size 1) (drill 0.5) (layers F.Cu B.Cu) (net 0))
 (via (at 150.495 67.31) (size 1) (drill 0.5) (layers F.Cu B.Cu) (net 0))
 (via (at 129.54 65.405) (size 1) (drill 0.5) (layers F.Cu B.Cu) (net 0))
 (via (at 132.08 65.405) (size 1) (drill 0.5) (layers F.Cu B.Cu) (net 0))
 (via (at 133.35 65.405) (size 1) (drill 0.5) (layers F.Cu B.Cu) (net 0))
 (via (at 134.62 65.405) (size 1) (drill 0.5) (layers F.Cu B.Cu) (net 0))
 (via (at 135.89 65.405) (size 1) (drill 0.5) (layers F.Cu B.Cu) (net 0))
 (via (at 137.16 65.405) (size 1) (drill 0.5) (layers F.Cu B.Cu) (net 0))
 (via (at 138.43 65.405) (size 1) (drill 0.5) (layers F.Cu B.Cu) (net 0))
 (via (at 139.7 65.405) (size 1) (drill 0.5) (layers F.Cu B.Cu) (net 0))
 (via (at 140.97 65.405) (size 1) (drill 0.5) (layers F.Cu B.Cu) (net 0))
 (via (at 142.24 65.405) (size 1) (drill 0.5) (layers F.Cu B.Cu) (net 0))
 (via (at 143.51 65.405) (size 1) (drill 0.5) (layers F.Cu B.Cu) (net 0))
 (via (at 144.78 65.405) (size 1) (drill 0.5) (layers F.Cu B.Cu) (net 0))
 (via (at 146.05 65.405) (size 1) (drill 0.5) (layers F.Cu B.Cu) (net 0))
 (via (at 147.32 65.405) (size 1) (drill 0.5) (layers F.Cu B.Cu) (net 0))
 (via (at 148.59 65.405) (size 1) (drill 0.5) (layers F.Cu B.Cu) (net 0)))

